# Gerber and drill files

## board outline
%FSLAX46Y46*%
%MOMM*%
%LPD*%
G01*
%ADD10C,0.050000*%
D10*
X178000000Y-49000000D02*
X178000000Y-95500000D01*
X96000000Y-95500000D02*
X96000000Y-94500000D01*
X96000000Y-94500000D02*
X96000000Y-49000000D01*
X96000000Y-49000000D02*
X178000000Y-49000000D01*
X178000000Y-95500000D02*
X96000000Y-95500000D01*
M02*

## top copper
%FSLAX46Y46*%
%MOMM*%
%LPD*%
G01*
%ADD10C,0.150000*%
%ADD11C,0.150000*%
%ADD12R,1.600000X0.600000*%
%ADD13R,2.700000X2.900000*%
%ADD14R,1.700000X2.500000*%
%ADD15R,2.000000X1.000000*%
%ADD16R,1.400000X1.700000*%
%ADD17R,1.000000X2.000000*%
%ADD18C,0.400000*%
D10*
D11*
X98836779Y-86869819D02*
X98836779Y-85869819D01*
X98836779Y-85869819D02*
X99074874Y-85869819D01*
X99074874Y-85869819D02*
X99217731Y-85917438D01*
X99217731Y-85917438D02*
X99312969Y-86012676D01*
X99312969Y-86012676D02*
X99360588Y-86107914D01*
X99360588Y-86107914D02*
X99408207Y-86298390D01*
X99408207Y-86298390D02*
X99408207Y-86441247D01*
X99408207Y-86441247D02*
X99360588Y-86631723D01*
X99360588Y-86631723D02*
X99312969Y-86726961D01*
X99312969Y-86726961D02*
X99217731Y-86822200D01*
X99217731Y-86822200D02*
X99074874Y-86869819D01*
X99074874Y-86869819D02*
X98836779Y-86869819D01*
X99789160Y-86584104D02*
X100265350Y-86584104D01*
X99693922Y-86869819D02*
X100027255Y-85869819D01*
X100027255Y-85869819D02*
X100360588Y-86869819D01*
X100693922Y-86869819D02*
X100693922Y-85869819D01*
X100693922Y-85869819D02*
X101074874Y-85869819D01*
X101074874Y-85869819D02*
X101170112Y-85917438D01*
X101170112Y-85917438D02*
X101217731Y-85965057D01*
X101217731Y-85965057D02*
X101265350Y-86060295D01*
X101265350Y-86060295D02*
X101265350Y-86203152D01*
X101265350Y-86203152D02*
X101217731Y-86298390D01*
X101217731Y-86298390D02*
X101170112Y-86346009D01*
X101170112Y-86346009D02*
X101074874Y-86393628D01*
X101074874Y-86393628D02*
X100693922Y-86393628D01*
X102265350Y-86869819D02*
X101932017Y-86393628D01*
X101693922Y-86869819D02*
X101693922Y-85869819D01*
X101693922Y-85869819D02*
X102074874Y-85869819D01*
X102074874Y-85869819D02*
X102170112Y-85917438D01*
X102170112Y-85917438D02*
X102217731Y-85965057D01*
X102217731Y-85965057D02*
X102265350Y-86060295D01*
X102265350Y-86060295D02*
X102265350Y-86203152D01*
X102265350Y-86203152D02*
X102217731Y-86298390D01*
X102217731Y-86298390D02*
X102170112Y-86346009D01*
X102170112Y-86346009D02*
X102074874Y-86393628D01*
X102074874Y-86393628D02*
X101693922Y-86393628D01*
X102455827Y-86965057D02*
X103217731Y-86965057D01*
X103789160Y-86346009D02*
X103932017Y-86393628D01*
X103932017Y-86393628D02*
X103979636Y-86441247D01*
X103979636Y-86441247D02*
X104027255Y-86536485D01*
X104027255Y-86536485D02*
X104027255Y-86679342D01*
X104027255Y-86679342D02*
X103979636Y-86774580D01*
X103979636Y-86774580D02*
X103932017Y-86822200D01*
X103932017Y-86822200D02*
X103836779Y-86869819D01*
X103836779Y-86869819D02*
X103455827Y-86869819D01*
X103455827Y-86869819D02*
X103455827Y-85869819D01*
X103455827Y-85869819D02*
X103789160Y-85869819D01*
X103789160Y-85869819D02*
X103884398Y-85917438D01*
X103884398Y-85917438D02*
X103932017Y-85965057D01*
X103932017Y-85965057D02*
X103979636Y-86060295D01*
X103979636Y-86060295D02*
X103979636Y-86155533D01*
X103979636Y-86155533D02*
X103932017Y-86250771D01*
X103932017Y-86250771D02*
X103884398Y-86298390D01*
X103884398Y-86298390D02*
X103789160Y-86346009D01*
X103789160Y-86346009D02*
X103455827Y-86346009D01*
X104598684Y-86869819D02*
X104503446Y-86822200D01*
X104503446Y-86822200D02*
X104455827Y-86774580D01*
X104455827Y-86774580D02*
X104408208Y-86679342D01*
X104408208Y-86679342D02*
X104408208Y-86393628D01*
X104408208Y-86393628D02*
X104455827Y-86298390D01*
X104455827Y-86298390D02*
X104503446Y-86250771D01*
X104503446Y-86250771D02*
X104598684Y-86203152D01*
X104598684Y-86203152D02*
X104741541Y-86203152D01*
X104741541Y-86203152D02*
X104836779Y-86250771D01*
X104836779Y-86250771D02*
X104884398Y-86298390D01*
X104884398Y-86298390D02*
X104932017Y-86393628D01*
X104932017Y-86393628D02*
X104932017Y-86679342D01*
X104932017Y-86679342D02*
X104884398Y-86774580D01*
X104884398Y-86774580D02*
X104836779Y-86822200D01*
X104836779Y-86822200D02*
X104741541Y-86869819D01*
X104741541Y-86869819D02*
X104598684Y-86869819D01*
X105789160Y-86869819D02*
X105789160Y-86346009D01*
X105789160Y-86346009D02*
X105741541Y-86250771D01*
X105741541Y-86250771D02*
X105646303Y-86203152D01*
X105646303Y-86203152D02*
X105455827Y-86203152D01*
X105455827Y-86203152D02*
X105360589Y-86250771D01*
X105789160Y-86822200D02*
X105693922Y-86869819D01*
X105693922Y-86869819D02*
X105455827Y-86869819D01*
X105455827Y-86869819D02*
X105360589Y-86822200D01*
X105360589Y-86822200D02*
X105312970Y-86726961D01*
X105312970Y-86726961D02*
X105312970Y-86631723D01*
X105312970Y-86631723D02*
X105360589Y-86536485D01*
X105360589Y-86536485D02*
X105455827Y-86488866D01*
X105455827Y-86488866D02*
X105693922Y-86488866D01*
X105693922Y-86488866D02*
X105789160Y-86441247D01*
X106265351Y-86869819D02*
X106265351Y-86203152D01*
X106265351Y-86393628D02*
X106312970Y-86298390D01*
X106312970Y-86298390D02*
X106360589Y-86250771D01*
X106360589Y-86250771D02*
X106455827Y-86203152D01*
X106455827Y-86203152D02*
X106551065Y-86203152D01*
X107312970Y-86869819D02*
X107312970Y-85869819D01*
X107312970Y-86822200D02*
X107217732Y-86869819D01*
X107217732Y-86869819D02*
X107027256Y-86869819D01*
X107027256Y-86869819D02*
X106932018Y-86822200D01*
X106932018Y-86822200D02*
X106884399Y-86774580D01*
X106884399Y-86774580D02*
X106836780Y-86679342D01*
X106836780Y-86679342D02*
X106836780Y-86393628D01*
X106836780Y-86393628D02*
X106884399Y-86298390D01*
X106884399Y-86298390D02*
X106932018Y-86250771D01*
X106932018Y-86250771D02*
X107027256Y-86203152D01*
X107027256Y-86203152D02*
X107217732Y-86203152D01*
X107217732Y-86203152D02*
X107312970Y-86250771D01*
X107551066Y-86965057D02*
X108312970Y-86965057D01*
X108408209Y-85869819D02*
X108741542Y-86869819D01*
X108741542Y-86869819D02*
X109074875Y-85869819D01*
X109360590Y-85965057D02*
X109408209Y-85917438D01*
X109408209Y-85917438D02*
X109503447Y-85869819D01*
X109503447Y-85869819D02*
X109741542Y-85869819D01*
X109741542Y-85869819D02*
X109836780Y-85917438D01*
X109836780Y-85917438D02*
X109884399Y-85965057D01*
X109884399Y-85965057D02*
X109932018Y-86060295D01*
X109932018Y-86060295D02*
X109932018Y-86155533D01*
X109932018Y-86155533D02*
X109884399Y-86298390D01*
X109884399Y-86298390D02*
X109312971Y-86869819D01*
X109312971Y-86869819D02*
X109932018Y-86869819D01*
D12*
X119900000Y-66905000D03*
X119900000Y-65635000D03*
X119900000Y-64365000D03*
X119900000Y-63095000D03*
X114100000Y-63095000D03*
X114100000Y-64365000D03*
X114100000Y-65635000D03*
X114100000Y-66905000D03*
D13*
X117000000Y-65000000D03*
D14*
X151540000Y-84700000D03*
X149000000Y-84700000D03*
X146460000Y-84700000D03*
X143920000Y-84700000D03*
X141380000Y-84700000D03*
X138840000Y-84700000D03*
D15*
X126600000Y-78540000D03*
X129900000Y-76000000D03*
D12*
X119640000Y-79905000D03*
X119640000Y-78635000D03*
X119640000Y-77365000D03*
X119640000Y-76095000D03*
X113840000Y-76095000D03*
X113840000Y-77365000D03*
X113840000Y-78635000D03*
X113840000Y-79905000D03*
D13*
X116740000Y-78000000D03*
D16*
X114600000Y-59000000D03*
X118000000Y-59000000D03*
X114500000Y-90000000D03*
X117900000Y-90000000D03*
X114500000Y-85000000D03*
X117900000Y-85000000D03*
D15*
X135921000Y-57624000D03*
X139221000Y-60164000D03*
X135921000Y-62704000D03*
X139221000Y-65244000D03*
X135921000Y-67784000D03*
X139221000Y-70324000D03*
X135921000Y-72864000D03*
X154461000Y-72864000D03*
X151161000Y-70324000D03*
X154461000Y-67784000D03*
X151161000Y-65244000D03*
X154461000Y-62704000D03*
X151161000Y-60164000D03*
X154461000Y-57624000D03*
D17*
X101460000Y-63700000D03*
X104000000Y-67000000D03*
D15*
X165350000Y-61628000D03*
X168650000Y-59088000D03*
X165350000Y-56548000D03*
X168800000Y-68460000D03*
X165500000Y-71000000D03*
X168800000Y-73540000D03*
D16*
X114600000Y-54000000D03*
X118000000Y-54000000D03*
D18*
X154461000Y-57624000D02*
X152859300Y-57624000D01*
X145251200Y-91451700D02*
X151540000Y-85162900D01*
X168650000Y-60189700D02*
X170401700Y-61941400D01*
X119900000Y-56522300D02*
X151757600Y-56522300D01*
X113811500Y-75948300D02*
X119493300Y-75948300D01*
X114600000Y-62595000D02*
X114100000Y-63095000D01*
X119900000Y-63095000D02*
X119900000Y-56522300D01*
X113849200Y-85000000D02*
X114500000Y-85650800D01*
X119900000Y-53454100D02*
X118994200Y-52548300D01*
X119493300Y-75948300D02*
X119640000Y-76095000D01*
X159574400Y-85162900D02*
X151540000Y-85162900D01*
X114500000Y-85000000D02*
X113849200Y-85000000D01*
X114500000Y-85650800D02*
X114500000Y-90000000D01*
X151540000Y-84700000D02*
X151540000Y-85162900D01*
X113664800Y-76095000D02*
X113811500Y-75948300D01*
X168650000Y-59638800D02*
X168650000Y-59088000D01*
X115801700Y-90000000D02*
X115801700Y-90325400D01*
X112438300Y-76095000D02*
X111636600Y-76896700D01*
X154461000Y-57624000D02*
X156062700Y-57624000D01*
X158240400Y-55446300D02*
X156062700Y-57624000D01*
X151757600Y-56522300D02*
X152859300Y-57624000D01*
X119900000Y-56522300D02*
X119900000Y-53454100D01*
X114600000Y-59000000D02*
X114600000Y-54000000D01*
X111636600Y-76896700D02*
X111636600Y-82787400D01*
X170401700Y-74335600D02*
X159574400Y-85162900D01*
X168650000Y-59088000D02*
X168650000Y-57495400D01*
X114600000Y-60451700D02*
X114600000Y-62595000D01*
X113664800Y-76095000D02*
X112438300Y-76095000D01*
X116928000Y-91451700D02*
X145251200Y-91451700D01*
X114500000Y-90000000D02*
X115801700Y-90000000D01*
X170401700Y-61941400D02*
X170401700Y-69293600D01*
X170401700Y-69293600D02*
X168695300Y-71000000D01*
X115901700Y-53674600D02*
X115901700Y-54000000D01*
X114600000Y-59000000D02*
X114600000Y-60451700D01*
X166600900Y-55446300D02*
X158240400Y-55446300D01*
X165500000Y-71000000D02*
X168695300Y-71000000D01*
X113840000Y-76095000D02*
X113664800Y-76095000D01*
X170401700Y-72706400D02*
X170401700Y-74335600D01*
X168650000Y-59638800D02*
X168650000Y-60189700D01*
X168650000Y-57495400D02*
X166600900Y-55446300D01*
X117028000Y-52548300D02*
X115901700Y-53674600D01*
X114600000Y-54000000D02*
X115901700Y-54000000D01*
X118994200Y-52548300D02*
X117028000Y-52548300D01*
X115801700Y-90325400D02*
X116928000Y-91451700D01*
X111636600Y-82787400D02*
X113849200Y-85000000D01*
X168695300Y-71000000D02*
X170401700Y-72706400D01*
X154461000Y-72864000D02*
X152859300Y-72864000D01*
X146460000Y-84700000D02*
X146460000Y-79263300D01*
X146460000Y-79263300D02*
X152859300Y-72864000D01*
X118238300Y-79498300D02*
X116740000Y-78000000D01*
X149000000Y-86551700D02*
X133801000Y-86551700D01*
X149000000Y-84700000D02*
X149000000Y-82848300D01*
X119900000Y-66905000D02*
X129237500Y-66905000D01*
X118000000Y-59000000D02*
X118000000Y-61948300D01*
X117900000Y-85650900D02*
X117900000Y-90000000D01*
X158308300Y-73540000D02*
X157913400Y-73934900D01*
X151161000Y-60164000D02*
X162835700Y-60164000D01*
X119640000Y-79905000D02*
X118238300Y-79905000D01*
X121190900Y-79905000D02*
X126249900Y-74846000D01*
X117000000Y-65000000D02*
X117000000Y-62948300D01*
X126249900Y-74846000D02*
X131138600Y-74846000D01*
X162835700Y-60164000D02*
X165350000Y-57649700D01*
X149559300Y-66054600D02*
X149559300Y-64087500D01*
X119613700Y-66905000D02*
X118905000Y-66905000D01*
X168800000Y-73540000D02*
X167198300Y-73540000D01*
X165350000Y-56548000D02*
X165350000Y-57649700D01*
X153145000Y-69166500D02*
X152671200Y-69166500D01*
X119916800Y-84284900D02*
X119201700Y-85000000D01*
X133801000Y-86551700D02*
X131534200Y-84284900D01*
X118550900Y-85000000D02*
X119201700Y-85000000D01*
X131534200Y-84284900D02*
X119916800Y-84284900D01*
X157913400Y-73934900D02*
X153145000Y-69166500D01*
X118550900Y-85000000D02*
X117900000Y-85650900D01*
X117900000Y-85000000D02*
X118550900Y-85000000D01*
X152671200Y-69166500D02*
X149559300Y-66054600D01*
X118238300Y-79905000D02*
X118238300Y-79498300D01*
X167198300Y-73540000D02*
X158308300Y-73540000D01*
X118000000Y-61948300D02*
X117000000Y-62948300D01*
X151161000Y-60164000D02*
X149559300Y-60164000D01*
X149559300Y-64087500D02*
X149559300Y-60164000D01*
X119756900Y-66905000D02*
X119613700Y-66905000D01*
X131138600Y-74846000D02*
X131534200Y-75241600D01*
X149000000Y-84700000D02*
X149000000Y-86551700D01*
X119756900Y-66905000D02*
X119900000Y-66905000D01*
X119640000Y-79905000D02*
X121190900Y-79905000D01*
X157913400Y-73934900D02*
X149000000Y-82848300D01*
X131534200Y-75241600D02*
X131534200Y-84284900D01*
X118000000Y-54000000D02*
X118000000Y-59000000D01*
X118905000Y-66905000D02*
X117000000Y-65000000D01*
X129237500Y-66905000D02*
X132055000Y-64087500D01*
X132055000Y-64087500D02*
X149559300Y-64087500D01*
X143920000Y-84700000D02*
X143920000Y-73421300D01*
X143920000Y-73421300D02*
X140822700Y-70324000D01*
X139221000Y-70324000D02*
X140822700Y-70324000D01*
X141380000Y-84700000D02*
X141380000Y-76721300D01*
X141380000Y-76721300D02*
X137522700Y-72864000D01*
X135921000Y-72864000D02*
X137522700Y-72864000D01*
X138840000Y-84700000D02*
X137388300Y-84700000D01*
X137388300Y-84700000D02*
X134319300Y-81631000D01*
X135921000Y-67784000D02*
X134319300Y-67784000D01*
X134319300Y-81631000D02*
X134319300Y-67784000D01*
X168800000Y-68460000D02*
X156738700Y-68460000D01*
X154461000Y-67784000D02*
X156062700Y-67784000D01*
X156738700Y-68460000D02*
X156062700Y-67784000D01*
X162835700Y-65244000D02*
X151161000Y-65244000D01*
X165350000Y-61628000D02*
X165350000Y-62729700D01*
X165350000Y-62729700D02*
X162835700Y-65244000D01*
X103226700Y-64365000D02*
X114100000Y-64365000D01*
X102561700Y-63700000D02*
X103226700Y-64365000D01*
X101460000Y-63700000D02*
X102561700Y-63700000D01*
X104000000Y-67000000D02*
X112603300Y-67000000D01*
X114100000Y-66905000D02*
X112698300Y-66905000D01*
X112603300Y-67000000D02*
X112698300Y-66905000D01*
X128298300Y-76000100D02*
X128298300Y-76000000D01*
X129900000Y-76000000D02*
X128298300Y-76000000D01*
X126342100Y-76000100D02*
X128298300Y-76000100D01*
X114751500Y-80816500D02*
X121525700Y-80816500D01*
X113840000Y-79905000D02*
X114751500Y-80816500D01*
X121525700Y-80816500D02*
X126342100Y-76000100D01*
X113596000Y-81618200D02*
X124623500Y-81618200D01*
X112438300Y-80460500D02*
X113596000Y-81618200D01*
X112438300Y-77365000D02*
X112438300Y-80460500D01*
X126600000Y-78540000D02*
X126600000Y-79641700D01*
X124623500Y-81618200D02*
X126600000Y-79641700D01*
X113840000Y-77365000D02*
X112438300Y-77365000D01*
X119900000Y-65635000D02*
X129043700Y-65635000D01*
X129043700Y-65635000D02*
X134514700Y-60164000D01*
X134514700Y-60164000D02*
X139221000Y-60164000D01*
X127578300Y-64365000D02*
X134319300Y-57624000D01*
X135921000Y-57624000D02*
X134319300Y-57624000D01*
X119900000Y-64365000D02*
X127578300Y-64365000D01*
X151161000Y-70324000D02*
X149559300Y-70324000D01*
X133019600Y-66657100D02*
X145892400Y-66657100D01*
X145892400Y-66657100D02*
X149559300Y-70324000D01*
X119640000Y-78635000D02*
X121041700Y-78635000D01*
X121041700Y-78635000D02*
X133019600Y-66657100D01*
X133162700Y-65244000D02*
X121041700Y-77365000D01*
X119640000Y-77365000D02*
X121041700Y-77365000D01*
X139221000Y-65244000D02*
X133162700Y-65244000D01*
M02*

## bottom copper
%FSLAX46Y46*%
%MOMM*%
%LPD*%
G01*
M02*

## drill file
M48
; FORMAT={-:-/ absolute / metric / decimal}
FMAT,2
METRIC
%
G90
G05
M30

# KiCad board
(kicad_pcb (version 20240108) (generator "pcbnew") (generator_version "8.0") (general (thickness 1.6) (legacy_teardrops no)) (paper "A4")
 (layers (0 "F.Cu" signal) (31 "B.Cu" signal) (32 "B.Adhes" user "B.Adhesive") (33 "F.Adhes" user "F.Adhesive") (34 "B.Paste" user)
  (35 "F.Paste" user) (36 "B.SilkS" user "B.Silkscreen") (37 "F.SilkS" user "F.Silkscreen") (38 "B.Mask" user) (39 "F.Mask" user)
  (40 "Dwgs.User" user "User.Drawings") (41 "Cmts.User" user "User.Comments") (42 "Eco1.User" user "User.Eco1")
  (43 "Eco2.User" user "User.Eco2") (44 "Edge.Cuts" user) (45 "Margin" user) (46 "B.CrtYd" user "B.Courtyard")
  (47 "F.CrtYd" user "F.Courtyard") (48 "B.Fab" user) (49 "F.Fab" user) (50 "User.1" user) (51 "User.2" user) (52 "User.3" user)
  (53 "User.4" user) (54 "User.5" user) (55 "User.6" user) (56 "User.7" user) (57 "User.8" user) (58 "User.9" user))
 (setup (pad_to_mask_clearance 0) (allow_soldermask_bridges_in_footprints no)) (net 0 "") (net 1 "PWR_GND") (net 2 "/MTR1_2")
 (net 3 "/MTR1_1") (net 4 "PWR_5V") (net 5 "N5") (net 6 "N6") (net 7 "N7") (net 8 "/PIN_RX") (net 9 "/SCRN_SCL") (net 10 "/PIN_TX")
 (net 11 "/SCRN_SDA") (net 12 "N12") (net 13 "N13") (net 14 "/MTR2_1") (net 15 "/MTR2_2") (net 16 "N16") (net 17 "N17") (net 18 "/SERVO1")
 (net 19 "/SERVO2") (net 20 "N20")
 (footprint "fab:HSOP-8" (layer "F.Cu") (at 117 65 180)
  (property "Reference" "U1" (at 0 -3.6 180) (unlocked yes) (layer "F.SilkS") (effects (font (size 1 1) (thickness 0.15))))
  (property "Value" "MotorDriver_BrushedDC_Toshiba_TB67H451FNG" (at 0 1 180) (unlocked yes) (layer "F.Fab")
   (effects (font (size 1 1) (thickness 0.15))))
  (pad "1" smd rect (at -2.9 -1.905 180) (size 1.6 0.6) (layers "F.Cu" "F.Paste" "F.Mask") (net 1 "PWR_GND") (thermal_bridge_angle 45))
  (pad "2" smd rect (at -2.9 -0.635 180) (size 1.6 0.6) (layers "F.Cu" "F.Paste" "F.Mask") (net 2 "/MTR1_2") (thermal_bridge_angle 45))
  (pad "3" smd rect (at -2.9 0.635 180) (size 1.6 0.6) (layers "F.Cu" "F.Paste" "F.Mask") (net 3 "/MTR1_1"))
  (pad "4" smd rect (at -2.9 1.905 180) (size 1.6 0.6) (layers "F.Cu" "F.Paste" "F.Mask") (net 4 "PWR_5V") (thermal_bridge_angle 45))
  (pad "5" smd rect (at 2.9 1.905 180) (size 1.6 0.6) (layers "F.Cu" "F.Paste" "F.Mask") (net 4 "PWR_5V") (thermal_bridge_angle 45))
  (pad "6" smd rect (at 2.9 0.635 180) (size 1.6 0.6) (layers "F.Cu" "F.Paste" "F.Mask") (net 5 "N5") (thermal_bridge_angle 45))
  (pad "7" smd rect (at 2.9 -0.635 180) (size 1.6 0.6) (layers "F.Cu" "F.Paste" "F.Mask") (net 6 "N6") (thermal_bridge_angle 45))
  (pad "8" smd rect (at 2.9 -1.905 180) (size 1.6 0.6) (layers "F.Cu" "F.Paste" "F.Mask") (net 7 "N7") (thermal_bridge_angle 45))
  (pad "9" smd rect (at 0 0 180) (size 2.7 2.9) (layers "F.Cu" "F.Paste" "F.Mask") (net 1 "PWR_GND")))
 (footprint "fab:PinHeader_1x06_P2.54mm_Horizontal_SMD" (layer "F.Cu") (at 151.54 84.7 -90)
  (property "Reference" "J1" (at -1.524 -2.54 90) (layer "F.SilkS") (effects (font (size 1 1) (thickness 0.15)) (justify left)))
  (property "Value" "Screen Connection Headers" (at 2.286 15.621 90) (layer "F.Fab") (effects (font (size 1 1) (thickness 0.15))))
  (pad "1" smd rect (at 0 0 270) (size 2.5 1.7) (layers "F.Cu" "F.Paste" "F.Mask") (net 4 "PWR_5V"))
  (pad "2" smd rect (at 0 2.54 270) (size 2.5 1.7) (layers "F.Cu" "F.Paste" "F.Mask") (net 1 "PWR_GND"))
  (pad "3" smd rect (at 0 5.08 270) (size 2.5 1.7) (layers "F.Cu" "F.Paste" "F.Mask") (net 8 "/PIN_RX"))
  (pad "4" smd rect (at 0 7.62 270) (size 2.5 1.7) (layers "F.Cu" "F.Paste" "F.Mask") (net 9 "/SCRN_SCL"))
  (pad "5" smd rect (at 0 10.16 270) (size 2.5 1.7) (layers "F.Cu" "F.Paste" "F.Mask") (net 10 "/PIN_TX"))
  (pad "6" smd rect (at 0 12.7 270) (size 2.5 1.7) (layers "F.Cu" "F.Paste" "F.Mask") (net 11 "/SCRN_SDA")))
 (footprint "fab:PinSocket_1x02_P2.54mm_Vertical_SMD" (layer "F.Cu") (at 128.25 77.27 180)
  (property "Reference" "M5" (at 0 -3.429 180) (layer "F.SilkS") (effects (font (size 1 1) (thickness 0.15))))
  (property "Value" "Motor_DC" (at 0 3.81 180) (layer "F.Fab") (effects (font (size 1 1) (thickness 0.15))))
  (pad "1" smd rect (at 1.65 -1.27 180) (size 2 1) (layers "F.Cu" "F.Paste" "F.Mask") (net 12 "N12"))
  (pad "2" smd rect (at -1.65 1.27 180) (size 2 1) (layers "F.Cu" "F.Paste" "F.Mask") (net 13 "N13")))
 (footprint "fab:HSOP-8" (layer "F.Cu") (at 116.74 78 180)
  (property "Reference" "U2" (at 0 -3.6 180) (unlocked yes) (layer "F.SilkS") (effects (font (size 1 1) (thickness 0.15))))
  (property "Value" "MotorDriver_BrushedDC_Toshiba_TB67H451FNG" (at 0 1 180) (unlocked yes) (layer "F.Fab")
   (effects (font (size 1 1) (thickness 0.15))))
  (pad "1" smd rect (at -2.9 -1.905 180) (size 1.6 0.6) (layers "F.Cu" "F.Paste" "F.Mask") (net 1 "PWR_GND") (thermal_bridge_angle 45))
  (pad "2" smd rect (at -2.9 -0.635 180) (size 1.6 0.6) (layers "F.Cu" "F.Paste" "F.Mask") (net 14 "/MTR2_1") (thermal_bridge_angle 45))
  (pad "3" smd rect (at -2.9 0.635 180) (size 1.6 0.6) (layers "F.Cu" "F.Paste" "F.Mask") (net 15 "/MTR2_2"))
  (pad "4" smd rect (at -2.9 1.905 180) (size 1.6 0.6) (layers "F.Cu" "F.Paste" "F.Mask") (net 4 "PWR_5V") (thermal_bridge_angle 45))
  (pad "5" smd rect (at 2.9 1.905 180) (size 1.6 0.6) (layers "F.Cu" "F.Paste" "F.Mask") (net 4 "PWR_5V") (thermal_bridge_angle 45))
  (pad "6" smd rect (at 2.9 0.635 180) (size 1.6 0.6) (layers "F.Cu" "F.Paste" "F.Mask") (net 12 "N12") (thermal_bridge_angle 45))
  (pad "7" smd rect (at 2.9 -0.635 180) (size 1.6 0.6) (layers "F.Cu" "F.Paste" "F.Mask") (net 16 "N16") (thermal_bridge_angle 45))
  (pad "8" smd rect (at 2.9 -1.905 180) (size 1.6 0.6) (layers "F.Cu" "F.Paste" "F.Mask") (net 13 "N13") (thermal_bridge_angle 45))
  (pad "9" smd rect (at 0 0 180) (size 2.7 2.9) (layers "F.Cu" "F.Paste" "F.Mask") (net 1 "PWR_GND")))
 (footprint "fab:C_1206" (layer "F.Cu") (at 116.3 59)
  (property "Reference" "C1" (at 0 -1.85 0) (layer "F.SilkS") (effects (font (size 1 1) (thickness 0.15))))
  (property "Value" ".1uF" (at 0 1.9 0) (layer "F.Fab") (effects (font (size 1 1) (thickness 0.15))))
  (pad "1" smd rect (at -1.7 0) (size 1.4 1.7) (layers "F.Cu" "F.Paste" "F.Mask") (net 4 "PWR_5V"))
  (pad "2" smd rect (at 1.7 0) (size 1.4 1.7) (layers "F.Cu" "F.Paste" "F.Mask") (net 1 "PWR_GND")))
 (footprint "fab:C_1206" (layer "F.Cu") (at 116.2 90)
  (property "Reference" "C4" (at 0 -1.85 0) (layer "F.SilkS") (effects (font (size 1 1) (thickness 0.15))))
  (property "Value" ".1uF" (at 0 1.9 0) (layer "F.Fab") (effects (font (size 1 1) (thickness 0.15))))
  (pad "1" smd rect (at -1.7 0) (size 1.4 1.7) (layers "F.Cu" "F.Paste" "F.Mask") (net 4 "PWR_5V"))
  (pad "2" smd rect (at 1.7 0) (size 1.4 1.7) (layers "F.Cu" "F.Paste" "F.Mask") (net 1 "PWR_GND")))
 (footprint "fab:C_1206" (layer "F.Cu") (at 116.2 85)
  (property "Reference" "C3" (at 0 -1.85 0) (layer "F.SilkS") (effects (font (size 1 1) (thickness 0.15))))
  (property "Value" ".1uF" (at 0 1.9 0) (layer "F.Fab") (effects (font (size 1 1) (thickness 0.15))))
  (pad "1" smd rect (at -1.7 0) (size 1.4 1.7) (layers "F.Cu" "F.Paste" "F.Mask") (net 4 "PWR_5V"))
  (pad "2" smd rect (at 1.7 0) (size 1.4 1.7) (layers "F.Cu" "F.Paste" "F.Mask") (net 1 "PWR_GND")))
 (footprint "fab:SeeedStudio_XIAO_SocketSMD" (layer "F.Cu") (at 145.191 65.244)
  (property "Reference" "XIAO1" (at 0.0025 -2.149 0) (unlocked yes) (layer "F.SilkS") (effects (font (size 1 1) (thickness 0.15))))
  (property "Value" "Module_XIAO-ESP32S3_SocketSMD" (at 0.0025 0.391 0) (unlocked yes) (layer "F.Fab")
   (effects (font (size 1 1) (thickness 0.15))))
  (pad "1" smd rect (at -9.27 -7.62) (size 2 1) (layers "F.Cu" "F.Paste" "F.Mask") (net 3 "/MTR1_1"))
  (pad "2" smd rect (at -5.97 -5.08) (size 2 1) (layers "F.Cu" "F.Paste" "F.Mask") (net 2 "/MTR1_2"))
  (pad "3" smd rect (at -9.27 -2.54) (size 2 1) (layers "F.Cu" "F.Paste" "F.Mask") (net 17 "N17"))
  (pad "4" smd rect (at -5.97 0) (size 2 1) (layers "F.Cu" "F.Paste" "F.Mask") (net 15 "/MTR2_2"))
  (pad "5" smd rect (at -9.27 2.54) (size 2 1) (layers "F.Cu" "F.Paste" "F.Mask") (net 11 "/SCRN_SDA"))
  (pad "6" smd rect (at -5.97 5.08) (size 2 1) (layers "F.Cu" "F.Paste" "F.Mask") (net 9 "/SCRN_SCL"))
  (pad "7" smd rect (at -9.27 7.62) (size 2 1) (layers "F.Cu" "F.Paste" "F.Mask") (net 10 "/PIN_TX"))
  (pad "8" smd rect (at 9.27 7.62) (size 2 1) (layers "F.Cu" "F.Paste" "F.Mask") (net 8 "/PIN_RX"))
  (pad "9" smd rect (at 5.97 5.08) (size 2 1) (layers "F.Cu" "F.Paste" "F.Mask") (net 14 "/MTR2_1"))
  (pad "10" smd rect (at 9.27 2.54) (size 2 1) (layers "F.Cu" "F.Paste" "F.Mask") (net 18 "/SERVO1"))
  (pad "11" smd rect (at 5.97 0) (size 2 1) (layers "F.Cu" "F.Paste" "F.Mask") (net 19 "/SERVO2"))
  (pad "12" smd rect (at 9.27 -2.54) (size 2 1) (layers "F.Cu" "F.Paste" "F.Mask") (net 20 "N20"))
  (pad "13" smd rect (at 5.97 -5.08) (size 2 1) (layers "F.Cu" "F.Paste" "F.Mask") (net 1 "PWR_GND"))
  (pad "14" smd rect (at 9.27 -7.62) (size 2 1) (layers "F.Cu" "F.Paste" "F.Mask") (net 4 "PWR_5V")))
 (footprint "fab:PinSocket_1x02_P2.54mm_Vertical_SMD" (layer "F.Cu") (at 102.73 65.35 90)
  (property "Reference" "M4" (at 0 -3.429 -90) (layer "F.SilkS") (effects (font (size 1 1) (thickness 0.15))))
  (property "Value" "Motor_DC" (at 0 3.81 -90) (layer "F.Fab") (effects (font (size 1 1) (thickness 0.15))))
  (pad "1" smd rect (at 1.65 -1.27 90) (size 2 1) (layers "F.Cu" "F.Paste" "F.Mask") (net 5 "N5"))
  (pad "2" smd rect (at -1.65 1.27 90) (size 2 1) (layers "F.Cu" "F.Paste" "F.Mask") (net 7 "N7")))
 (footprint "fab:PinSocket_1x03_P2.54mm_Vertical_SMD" (layer "F.Cu") (at 167 59.088 180)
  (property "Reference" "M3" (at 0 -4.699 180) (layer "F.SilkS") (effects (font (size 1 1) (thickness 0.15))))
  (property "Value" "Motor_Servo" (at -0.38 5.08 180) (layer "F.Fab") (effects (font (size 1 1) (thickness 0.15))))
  (pad "1" smd rect (at 1.65 -2.54 180) (size 2 1) (layers "F.Cu" "F.Paste" "F.Mask") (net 19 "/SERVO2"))
  (pad "2" smd rect (at -1.65 0 180) (size 2 1) (layers "F.Cu" "F.Paste" "F.Mask") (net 4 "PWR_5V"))
  (pad "3" smd rect (at 1.65 2.54 180) (size 2 1) (layers "F.Cu" "F.Paste" "F.Mask") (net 1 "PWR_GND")))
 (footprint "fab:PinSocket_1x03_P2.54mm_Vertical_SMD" (layer "F.Cu") (at 167.15 71)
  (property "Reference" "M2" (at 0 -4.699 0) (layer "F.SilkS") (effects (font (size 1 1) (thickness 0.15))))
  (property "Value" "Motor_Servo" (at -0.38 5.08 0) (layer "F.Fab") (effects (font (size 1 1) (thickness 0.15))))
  (pad "1" smd rect (at 1.65 -2.54) (size 2 1) (layers "F.Cu" "F.Paste" "F.Mask") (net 18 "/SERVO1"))
  (pad "2" smd rect (at -1.65 0) (size 2 1) (layers "F.Cu" "F.Paste" "F.Mask") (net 4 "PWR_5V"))
  (pad "3" smd rect (at 1.65 2.54) (size 2 1) (layers "F.Cu" "F.Paste" "F.Mask") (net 1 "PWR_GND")))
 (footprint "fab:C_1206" (layer "F.Cu") (at 116.3 54)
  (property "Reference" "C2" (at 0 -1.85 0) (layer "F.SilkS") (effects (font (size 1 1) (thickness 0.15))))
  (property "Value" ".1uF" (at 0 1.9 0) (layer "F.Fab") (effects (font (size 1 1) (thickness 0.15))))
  (pad "1" smd rect (at -1.7 0) (size 1.4 1.7) (layers "F.Cu" "F.Paste" "F.Mask") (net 4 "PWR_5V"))
  (pad "2" smd rect (at 1.7 0) (size 1.4 1.7) (layers "F.Cu" "F.Paste" "F.Mask") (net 1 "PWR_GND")))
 (gr_line (start 178 49) (end 178 95.5) (stroke (width 0.05) (type default)) (layer "Edge.Cuts"))
 (gr_line (start 96 95.5) (end 96 94.5) (stroke (width 0.05) (type default)) (layer "Edge.Cuts"))
 (gr_line (start 96 94.5) (end 96 49) (stroke (width 0.05) (type default)) (layer "Edge.Cuts"))
 (gr_line (start 96 49) (end 178 49) (stroke (width 0.05) (type default)) (layer "Edge.Cuts"))
 (gr_line (start 178 95.5) (end 96 95.5) (stroke (width 0.05) (type default)) (layer "Edge.Cuts"))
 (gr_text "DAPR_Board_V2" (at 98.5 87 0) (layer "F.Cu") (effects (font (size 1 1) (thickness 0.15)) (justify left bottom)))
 (segment (start 154.461 57.624) (end 152.8593 57.624) (width 0.4) (layer "F.Cu") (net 4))
 (segment (start 145.2512 91.4517) (end 151.54 85.1629) (width 0.4) (layer "F.Cu") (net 4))
 (segment (start 168.65 60.1897) (end 170.4017 61.9414) (width 0.4) (layer "F.Cu") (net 4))
 (segment (start 119.9 56.5223) (end 151.7576 56.5223) (width 0.4) (layer "F.Cu") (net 4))
 (segment (start 113.8115 75.9483) (end 119.4933 75.9483) (width 0.4) (layer "F.Cu") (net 4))
 (segment (start 114.6 62.595) (end 114.1 63.095) (width 0.4) (layer "F.Cu") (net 4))
 (segment (start 119.9 63.095) (end 119.9 56.5223) (width 0.4) (layer "F.Cu") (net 4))
 (segment (start 113.8492 85) (end 114.5 85.6508) (width 0.4) (layer "F.Cu") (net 4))
 (segment (start 119.9 53.4541) (end 118.9942 52.5483) (width 0.4) (layer "F.Cu") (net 4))
 (segment (start 119.4933 75.9483) (end 119.64 76.095) (width 0.4) (layer "F.Cu") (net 4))
 (segment (start 159.5744 85.1629) (end 151.54 85.1629) (width 0.4) (layer "F.Cu") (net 4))
 (segment (start 114.5 85) (end 113.8492 85) (width 0.4) (layer "F.Cu") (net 4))
 (segment (start 114.5 85.6508) (end 114.5 90) (width 0.4) (layer "F.Cu") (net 4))
 (segment (start 151.54 84.7) (end 151.54 85.1629) (width 0.4) (layer "F.Cu") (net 4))
 (segment (start 113.6648 76.095) (end 113.8115 75.9483) (width 0.4) (layer "F.Cu") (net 4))
 (segment (start 168.65 59.6388) (end 168.65 59.088) (width 0.4) (layer "F.Cu") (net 4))
 (segment (start 115.8017 90) (end 115.8017 90.3254) (width 0.4) (layer "F.Cu") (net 4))
 (segment (start 112.4383 76.095) (end 111.6366 76.8967) (width 0.4) (layer "F.Cu") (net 4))
 (segment (start 154.461 57.624) (end 156.0627 57.624) (width 0.4) (layer "F.Cu") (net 4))
 (segment (start 158.2404 55.4463) (end 156.0627 57.624) (width 0.4) (layer "F.Cu") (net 4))
 (segment (start 151.7576 56.5223) (end 152.8593 57.624) (width 0.4) (layer "F.Cu") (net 4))
 (segment (start 119.9 56.5223) (end 119.9 53.4541) (width 0.4) (layer "F.Cu") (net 4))
 (segment (start 114.6 59) (end 114.6 54) (width 0.4) (layer "F.Cu") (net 4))
 (segment (start 111.6366 76.8967) (end 111.6366 82.7874) (width 0.4) (layer "F.Cu") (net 4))
 (segment (start 170.4017 74.3356) (end 159.5744 85.1629) (width 0.4) (layer "F.Cu") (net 4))
 (segment (start 168.65 59.088) (end 168.65 57.4954) (width 0.4) (layer "F.Cu") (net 4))
 (segment (start 114.6 60.4517) (end 114.6 62.595) (width 0.4) (layer "F.Cu") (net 4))
 (segment (start 113.6648 76.095) (end 112.4383 76.095) (width 0.4) (layer "F.Cu") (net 4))
 (segment (start 116.928 91.4517) (end 145.2512 91.4517) (width 0.4) (layer "F.Cu") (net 4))
 (segment (start 114.5 90) (end 115.8017 90) (width 0.4) (layer "F.Cu") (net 4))
 (segment (start 170.4017 61.9414) (end 170.4017 69.2936) (width 0.4) (layer "F.Cu") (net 4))
 (segment (start 170.4017 69.2936) (end 168.6953 71) (width 0.4) (layer "F.Cu") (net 4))
 (segment (start 115.9017 53.6746) (end 115.9017 54) (width 0.4) (layer "F.Cu") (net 4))
 (segment (start 114.6 59) (end 114.6 60.4517) (width 0.4) (layer "F.Cu") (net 4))
 (segment (start 166.6009 55.4463) (end 158.2404 55.4463) (width 0.4) (layer "F.Cu") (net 4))
 (segment (start 165.5 71) (end 168.6953 71) (width 0.4) (layer "F.Cu") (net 4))
 (segment (start 113.84 76.095) (end 113.6648 76.095) (width 0.4) (layer "F.Cu") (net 4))
 (segment (start 170.4017 72.7064) (end 170.4017 74.3356) (width 0.4) (layer "F.Cu") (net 4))
 (segment (start 168.65 59.6388) (end 168.65 60.1897) (width 0.4) (layer "F.Cu") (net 4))
 (segment (start 168.65 57.4954) (end 166.6009 55.4463) (width 0.4) (layer "F.Cu") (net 4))
 (segment (start 117.028 52.5483) (end 115.9017 53.6746) (width 0.4) (layer "F.Cu") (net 4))
 (segment (start 114.6 54) (end 115.9017 54) (width 0.4) (layer "F.Cu") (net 4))
 (segment (start 118.9942 52.5483) (end 117.028 52.5483) (width 0.4) (layer "F.Cu") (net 4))
 (segment (start 115.8017 90.3254) (end 116.928 91.4517) (width 0.4) (layer "F.Cu") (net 4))
 (segment (start 111.6366 82.7874) (end 113.8492 85) (width 0.4) (layer "F.Cu") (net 4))
 (segment (start 168.6953 71) (end 170.4017 72.7064) (width 0.4) (layer "F.Cu") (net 4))
 (segment (start 154.461 72.864) (end 152.8593 72.864) (width 0.4) (layer "F.Cu") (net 8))
 (segment (start 146.46 84.7) (end 146.46 79.2633) (width 0.4) (layer "F.Cu") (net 8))
 (segment (start 146.46 79.2633) (end 152.8593 72.864) (width 0.4) (layer "F.Cu") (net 8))
 (segment (start 118.2383 79.4983) (end 116.74 78) (width 0.4) (layer "F.Cu") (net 1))
 (segment (start 149 86.5517) (end 133.801 86.5517) (width 0.4) (layer "F.Cu") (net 1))
 (segment (start 149 84.7) (end 149 82.8483) (width 0.4) (layer "F.Cu") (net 1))
 (segment (start 119.9 66.905) (end 129.2375 66.905) (width 0.4) (layer "F.Cu") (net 1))
 (segment (start 118 59) (end 118 61.9483) (width 0.4) (layer "F.Cu") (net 1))
 (segment (start 117.9 85.6509) (end 117.9 90) (width 0.4) (layer "F.Cu") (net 1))
 (segment (start 158.3083 73.54) (end 157.9134 73.9349) (width 0.4) (layer "F.Cu") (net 1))
 (segment (start 151.161 60.164) (end 162.8357 60.164) (width 0.4) (layer "F.Cu") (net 1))
 (segment (start 119.64 79.905) (end 118.2383 79.905) (width 0.4) (layer "F.Cu") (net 1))
 (segment (start 121.1909 79.905) (end 126.2499 74.846) (width 0.4) (layer "F.Cu") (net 1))
 (segment (start 117 65) (end 117 62.9483) (width 0.4) (layer "F.Cu") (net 1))
 (segment (start 126.2499 74.846) (end 131.1386 74.846) (width 0.4) (layer "F.Cu") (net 1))
 (segment (start 162.8357 60.164) (end 165.35 57.6497) (width 0.4) (layer "F.Cu") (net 1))
 (segment (start 149.5593 66.0546) (end 149.5593 64.0875) (width 0.4) (layer "F.Cu") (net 1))
 (segment (start 119.6137 66.905) (end 118.905 66.905) (width 0.4) (layer "F.Cu") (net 1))
 (segment (start 168.8 73.54) (end 167.1983 73.54) (width 0.4) (layer "F.Cu") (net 1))
 (segment (start 165.35 56.548) (end 165.35 57.6497) (width 0.4) (layer "F.Cu") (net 1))
 (segment (start 153.145 69.1665) (end 152.6712 69.1665) (width 0.4) (layer "F.Cu") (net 1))
 (segment (start 119.9168 84.2849) (end 119.2017 85) (width 0.4) (layer "F.Cu") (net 1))
 (segment (start 133.801 86.5517) (end 131.5342 84.2849) (width 0.4) (layer "F.Cu") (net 1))
 (segment (start 118.5509 85) (end 119.2017 85) (width 0.4) (layer "F.Cu") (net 1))
 (segment (start 131.5342 84.2849) (end 119.9168 84.2849) (width 0.4) (layer "F.Cu") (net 1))
 (segment (start 157.9134 73.9349) (end 153.145 69.1665) (width 0.4) (layer "F.Cu") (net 1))
 (segment (start 118.5509 85) (end 117.9 85.6509) (width 0.4) (layer "F.Cu") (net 1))
 (segment (start 117.9 85) (end 118.5509 85) (width 0.4) (layer "F.Cu") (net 1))
 (segment (start 152.6712 69.1665) (end 149.5593 66.0546) (width 0.4) (layer "F.Cu") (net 1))
 (segment (start 118.2383 79.905) (end 118.2383 79.4983) (width 0.4) (layer "F.Cu") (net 1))
 (segment (start 167.1983 73.54) (end 158.3083 73.54) (width 0.4) (layer "F.Cu") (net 1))
 (segment (start 118 61.9483) (end 117 62.9483) (width 0.4) (layer "F.Cu") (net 1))
 (segment (start 151.161 60.164) (end 149.5593 60.164) (width 0.4) (layer "F.Cu") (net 1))
 (segment (start 149.5593 64.0875) (end 149.5593 60.164) (width 0.4) (layer "F.Cu") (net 1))
 (segment (start 119.7569 66.905) (end 119.6137 66.905) (width 0.4) (layer "F.Cu") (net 1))
 (segment (start 131.1386 74.846) (end 131.5342 75.2416) (width 0.4) (layer "F.Cu") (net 1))
 (segment (start 149 84.7) (end 149 86.5517) (width 0.4) (layer "F.Cu") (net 1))
 (segment (start 119.7569 66.905) (end 119.9 66.905) (width 0.4) (layer "F.Cu") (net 1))
 (segment (start 119.64 79.905) (end 121.1909 79.905) (width 0.4) (layer "F.Cu") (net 1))
 (segment (start 157.9134 73.9349) (end 149 82.8483) (width 0.4) (layer "F.Cu") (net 1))
 (segment (start 131.5342 75.2416) (end 131.5342 84.2849) (width 0.4) (layer "F.Cu") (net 1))
 (segment (start 118 54) (end 118 59) (width 0.4) (layer "F.Cu") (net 1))
 (segment (start 118.905 66.905) (end 117 65) (width 0.4) (layer "F.Cu") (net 1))
 (segment (start 129.2375 66.905) (end 132.055 64.0875) (width 0.4) (layer "F.Cu") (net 1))
 (segment (start 132.055 64.0875) (end 149.5593 64.0875) (width 0.4) (layer "F.Cu") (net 1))
 (segment (start 143.92 84.7) (end 143.92 73.4213) (width 0.4) (layer "F.Cu") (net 9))
 (segment (start 143.92 73.4213) (end 140.8227 70.324) (width 0.4) (layer "F.Cu") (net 9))
 (segment (start 139.221 70.324) (end 140.8227 70.324) (width 0.4) (layer "F.Cu") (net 9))
 (segment (start 141.38 84.7) (end 141.38 76.7213) (width 0.4) (layer "F.Cu") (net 10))
 (segment (start 141.38 76.7213) (end 137.5227 72.864) (width 0.4) (layer "F.Cu") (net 10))
 (segment (start 135.921 72.864) (end 137.5227 72.864) (width 0.4) (layer "F.Cu") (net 10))
 (segment (start 138.84 84.7) (end 137.3883 84.7) (width 0.4) (layer "F.Cu") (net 11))
 (segment (start 137.3883 84.7) (end 134.3193 81.631) (width 0.4) (layer "F.Cu") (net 11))
 (segment (start 135.921 67.784) (end 134.3193 67.784) (width 0.4) (layer "F.Cu") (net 11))
 (segment (start 134.3193 81.631) (end 134.3193 67.784) (width 0.4) (layer "F.Cu") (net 11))
 (segment (start 168.8 68.46) (end 156.7387 68.46) (width 0.4) (layer "F.Cu") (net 18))
 (segment (start 154.461 67.784) (end 156.0627 67.784) (width 0.4) (layer "F.Cu") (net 18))
 (segment (start 156.7387 68.46) (end 156.0627 67.784) (width 0.4) (layer "F.Cu") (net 18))
 (segment (start 162.8357 65.244) (end 151.161 65.244) (width 0.4) (layer "F.Cu") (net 19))
 (segment (start 165.35 61.628) (end 165.35 62.7297) (width 0.4) (layer "F.Cu") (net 19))
 (segment (start 165.35 62.7297) (end 162.8357 65.244) (width 0.4) (layer "F.Cu") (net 19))
 (segment (start 103.2267 64.365) (end 114.1 64.365) (width 0.4) (layer "F.Cu") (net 5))
 (segment (start 102.5617 63.7) (end 103.2267 64.365) (width 0.4) (layer "F.Cu") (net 5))
 (segment (start 101.46 63.7) (end 102.5617 63.7) (width 0.4) (layer "F.Cu") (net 5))
 (segment (start 104 67) (end 112.6033 67) (width 0.4) (layer "F.Cu") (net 7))
 (segment (start 114.1 66.905) (end 112.6983 66.905) (width 0.4) (layer "F.Cu") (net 7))
 (segment (start 112.6033 67) (end 112.6983 66.905) (width 0.4) (layer "F.Cu") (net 7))
 (segment (start 128.2983 76.0001) (end 128.2983 76) (width 0.4) (layer "F.Cu") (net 13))
 (segment (start 129.9 76) (end 128.2983 76) (width 0.4) (layer "F.Cu") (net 13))
 (segment (start 126.3421 76.0001) (end 128.2983 76.0001) (width 0.4) (layer "F.Cu") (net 13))
 (segment (start 114.7515 80.8165) (end 121.5257 80.8165) (width 0.4) (layer "F.Cu") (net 13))
 (segment (start 113.84 79.905) (end 114.7515 80.8165) (width 0.4) (layer "F.Cu") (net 13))
 (segment (start 121.5257 80.8165) (end 126.3421 76.0001) (width 0.4) (layer "F.Cu") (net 13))
 (segment (start 113.596 81.6182) (end 124.6235 81.6182) (width 0.4) (layer "F.Cu") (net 12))
 (segment (start 112.4383 80.4605) (end 113.596 81.6182) (width 0.4) (layer "F.Cu") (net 12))
 (segment (start 112.4383 77.365) (end 112.4383 80.4605) (width 0.4) (layer "F.Cu") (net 12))
 (segment (start 126.6 78.54) (end 126.6 79.6417) (width 0.4) (layer "F.Cu") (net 12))
 (segment (start 124.6235 81.6182) (end 126.6 79.6417) (width 0.4) (layer "F.Cu") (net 12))
 (segment (start 113.84 77.365) (end 112.4383 77.365) (width 0.4) (layer "F.Cu") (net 12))
 (segment (start 119.9 65.635) (end 129.0437 65.635) (width 0.4) (layer "F.Cu") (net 2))
 (segment (start 129.0437 65.635) (end 134.5147 60.164) (width 0.4) (layer "F.Cu") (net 2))
 (segment (start 134.5147 60.164) (end 139.221 60.164) (width 0.4) (layer "F.Cu") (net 2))
 (segment (start 127.5783 64.365) (end 134.3193 57.624) (width 0.4) (layer "F.Cu") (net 3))
 (segment (start 135.921 57.624) (end 134.3193 57.624) (width 0.4) (layer "F.Cu") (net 3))
 (segment (start 119.9 64.365) (end 127.5783 64.365) (width 0.4) (layer "F.Cu") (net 3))
 (segment (start 151.161 70.324) (end 149.5593 70.324) (width 0.4) (layer "F.Cu") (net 14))
 (segment (start 133.0196 66.6571) (end 145.8924 66.6571) (width 0.4) (layer "F.Cu") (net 14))
 (segment (start 145.8924 66.6571) (end 149.5593 70.324) (width 0.4) (layer "F.Cu") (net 14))
 (segment (start 119.64 78.635) (end 121.0417 78.635) (width 0.4) (layer "F.Cu") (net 14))
 (segment (start 121.0417 78.635) (end 133.0196 66.6571) (width 0.4) (layer "F.Cu") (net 14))
 (segment (start 133.1627 65.244) (end 121.0417 77.365) (width 0.4) (layer "F.Cu") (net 15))
 (segment (start 119.64 77.365) (end 121.0417 77.365) (width 0.4) (layer "F.Cu") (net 15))
 (segment (start 139.221 65.244) (end 133.1627 65.244) (width 0.4) (layer "F.Cu") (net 15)))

